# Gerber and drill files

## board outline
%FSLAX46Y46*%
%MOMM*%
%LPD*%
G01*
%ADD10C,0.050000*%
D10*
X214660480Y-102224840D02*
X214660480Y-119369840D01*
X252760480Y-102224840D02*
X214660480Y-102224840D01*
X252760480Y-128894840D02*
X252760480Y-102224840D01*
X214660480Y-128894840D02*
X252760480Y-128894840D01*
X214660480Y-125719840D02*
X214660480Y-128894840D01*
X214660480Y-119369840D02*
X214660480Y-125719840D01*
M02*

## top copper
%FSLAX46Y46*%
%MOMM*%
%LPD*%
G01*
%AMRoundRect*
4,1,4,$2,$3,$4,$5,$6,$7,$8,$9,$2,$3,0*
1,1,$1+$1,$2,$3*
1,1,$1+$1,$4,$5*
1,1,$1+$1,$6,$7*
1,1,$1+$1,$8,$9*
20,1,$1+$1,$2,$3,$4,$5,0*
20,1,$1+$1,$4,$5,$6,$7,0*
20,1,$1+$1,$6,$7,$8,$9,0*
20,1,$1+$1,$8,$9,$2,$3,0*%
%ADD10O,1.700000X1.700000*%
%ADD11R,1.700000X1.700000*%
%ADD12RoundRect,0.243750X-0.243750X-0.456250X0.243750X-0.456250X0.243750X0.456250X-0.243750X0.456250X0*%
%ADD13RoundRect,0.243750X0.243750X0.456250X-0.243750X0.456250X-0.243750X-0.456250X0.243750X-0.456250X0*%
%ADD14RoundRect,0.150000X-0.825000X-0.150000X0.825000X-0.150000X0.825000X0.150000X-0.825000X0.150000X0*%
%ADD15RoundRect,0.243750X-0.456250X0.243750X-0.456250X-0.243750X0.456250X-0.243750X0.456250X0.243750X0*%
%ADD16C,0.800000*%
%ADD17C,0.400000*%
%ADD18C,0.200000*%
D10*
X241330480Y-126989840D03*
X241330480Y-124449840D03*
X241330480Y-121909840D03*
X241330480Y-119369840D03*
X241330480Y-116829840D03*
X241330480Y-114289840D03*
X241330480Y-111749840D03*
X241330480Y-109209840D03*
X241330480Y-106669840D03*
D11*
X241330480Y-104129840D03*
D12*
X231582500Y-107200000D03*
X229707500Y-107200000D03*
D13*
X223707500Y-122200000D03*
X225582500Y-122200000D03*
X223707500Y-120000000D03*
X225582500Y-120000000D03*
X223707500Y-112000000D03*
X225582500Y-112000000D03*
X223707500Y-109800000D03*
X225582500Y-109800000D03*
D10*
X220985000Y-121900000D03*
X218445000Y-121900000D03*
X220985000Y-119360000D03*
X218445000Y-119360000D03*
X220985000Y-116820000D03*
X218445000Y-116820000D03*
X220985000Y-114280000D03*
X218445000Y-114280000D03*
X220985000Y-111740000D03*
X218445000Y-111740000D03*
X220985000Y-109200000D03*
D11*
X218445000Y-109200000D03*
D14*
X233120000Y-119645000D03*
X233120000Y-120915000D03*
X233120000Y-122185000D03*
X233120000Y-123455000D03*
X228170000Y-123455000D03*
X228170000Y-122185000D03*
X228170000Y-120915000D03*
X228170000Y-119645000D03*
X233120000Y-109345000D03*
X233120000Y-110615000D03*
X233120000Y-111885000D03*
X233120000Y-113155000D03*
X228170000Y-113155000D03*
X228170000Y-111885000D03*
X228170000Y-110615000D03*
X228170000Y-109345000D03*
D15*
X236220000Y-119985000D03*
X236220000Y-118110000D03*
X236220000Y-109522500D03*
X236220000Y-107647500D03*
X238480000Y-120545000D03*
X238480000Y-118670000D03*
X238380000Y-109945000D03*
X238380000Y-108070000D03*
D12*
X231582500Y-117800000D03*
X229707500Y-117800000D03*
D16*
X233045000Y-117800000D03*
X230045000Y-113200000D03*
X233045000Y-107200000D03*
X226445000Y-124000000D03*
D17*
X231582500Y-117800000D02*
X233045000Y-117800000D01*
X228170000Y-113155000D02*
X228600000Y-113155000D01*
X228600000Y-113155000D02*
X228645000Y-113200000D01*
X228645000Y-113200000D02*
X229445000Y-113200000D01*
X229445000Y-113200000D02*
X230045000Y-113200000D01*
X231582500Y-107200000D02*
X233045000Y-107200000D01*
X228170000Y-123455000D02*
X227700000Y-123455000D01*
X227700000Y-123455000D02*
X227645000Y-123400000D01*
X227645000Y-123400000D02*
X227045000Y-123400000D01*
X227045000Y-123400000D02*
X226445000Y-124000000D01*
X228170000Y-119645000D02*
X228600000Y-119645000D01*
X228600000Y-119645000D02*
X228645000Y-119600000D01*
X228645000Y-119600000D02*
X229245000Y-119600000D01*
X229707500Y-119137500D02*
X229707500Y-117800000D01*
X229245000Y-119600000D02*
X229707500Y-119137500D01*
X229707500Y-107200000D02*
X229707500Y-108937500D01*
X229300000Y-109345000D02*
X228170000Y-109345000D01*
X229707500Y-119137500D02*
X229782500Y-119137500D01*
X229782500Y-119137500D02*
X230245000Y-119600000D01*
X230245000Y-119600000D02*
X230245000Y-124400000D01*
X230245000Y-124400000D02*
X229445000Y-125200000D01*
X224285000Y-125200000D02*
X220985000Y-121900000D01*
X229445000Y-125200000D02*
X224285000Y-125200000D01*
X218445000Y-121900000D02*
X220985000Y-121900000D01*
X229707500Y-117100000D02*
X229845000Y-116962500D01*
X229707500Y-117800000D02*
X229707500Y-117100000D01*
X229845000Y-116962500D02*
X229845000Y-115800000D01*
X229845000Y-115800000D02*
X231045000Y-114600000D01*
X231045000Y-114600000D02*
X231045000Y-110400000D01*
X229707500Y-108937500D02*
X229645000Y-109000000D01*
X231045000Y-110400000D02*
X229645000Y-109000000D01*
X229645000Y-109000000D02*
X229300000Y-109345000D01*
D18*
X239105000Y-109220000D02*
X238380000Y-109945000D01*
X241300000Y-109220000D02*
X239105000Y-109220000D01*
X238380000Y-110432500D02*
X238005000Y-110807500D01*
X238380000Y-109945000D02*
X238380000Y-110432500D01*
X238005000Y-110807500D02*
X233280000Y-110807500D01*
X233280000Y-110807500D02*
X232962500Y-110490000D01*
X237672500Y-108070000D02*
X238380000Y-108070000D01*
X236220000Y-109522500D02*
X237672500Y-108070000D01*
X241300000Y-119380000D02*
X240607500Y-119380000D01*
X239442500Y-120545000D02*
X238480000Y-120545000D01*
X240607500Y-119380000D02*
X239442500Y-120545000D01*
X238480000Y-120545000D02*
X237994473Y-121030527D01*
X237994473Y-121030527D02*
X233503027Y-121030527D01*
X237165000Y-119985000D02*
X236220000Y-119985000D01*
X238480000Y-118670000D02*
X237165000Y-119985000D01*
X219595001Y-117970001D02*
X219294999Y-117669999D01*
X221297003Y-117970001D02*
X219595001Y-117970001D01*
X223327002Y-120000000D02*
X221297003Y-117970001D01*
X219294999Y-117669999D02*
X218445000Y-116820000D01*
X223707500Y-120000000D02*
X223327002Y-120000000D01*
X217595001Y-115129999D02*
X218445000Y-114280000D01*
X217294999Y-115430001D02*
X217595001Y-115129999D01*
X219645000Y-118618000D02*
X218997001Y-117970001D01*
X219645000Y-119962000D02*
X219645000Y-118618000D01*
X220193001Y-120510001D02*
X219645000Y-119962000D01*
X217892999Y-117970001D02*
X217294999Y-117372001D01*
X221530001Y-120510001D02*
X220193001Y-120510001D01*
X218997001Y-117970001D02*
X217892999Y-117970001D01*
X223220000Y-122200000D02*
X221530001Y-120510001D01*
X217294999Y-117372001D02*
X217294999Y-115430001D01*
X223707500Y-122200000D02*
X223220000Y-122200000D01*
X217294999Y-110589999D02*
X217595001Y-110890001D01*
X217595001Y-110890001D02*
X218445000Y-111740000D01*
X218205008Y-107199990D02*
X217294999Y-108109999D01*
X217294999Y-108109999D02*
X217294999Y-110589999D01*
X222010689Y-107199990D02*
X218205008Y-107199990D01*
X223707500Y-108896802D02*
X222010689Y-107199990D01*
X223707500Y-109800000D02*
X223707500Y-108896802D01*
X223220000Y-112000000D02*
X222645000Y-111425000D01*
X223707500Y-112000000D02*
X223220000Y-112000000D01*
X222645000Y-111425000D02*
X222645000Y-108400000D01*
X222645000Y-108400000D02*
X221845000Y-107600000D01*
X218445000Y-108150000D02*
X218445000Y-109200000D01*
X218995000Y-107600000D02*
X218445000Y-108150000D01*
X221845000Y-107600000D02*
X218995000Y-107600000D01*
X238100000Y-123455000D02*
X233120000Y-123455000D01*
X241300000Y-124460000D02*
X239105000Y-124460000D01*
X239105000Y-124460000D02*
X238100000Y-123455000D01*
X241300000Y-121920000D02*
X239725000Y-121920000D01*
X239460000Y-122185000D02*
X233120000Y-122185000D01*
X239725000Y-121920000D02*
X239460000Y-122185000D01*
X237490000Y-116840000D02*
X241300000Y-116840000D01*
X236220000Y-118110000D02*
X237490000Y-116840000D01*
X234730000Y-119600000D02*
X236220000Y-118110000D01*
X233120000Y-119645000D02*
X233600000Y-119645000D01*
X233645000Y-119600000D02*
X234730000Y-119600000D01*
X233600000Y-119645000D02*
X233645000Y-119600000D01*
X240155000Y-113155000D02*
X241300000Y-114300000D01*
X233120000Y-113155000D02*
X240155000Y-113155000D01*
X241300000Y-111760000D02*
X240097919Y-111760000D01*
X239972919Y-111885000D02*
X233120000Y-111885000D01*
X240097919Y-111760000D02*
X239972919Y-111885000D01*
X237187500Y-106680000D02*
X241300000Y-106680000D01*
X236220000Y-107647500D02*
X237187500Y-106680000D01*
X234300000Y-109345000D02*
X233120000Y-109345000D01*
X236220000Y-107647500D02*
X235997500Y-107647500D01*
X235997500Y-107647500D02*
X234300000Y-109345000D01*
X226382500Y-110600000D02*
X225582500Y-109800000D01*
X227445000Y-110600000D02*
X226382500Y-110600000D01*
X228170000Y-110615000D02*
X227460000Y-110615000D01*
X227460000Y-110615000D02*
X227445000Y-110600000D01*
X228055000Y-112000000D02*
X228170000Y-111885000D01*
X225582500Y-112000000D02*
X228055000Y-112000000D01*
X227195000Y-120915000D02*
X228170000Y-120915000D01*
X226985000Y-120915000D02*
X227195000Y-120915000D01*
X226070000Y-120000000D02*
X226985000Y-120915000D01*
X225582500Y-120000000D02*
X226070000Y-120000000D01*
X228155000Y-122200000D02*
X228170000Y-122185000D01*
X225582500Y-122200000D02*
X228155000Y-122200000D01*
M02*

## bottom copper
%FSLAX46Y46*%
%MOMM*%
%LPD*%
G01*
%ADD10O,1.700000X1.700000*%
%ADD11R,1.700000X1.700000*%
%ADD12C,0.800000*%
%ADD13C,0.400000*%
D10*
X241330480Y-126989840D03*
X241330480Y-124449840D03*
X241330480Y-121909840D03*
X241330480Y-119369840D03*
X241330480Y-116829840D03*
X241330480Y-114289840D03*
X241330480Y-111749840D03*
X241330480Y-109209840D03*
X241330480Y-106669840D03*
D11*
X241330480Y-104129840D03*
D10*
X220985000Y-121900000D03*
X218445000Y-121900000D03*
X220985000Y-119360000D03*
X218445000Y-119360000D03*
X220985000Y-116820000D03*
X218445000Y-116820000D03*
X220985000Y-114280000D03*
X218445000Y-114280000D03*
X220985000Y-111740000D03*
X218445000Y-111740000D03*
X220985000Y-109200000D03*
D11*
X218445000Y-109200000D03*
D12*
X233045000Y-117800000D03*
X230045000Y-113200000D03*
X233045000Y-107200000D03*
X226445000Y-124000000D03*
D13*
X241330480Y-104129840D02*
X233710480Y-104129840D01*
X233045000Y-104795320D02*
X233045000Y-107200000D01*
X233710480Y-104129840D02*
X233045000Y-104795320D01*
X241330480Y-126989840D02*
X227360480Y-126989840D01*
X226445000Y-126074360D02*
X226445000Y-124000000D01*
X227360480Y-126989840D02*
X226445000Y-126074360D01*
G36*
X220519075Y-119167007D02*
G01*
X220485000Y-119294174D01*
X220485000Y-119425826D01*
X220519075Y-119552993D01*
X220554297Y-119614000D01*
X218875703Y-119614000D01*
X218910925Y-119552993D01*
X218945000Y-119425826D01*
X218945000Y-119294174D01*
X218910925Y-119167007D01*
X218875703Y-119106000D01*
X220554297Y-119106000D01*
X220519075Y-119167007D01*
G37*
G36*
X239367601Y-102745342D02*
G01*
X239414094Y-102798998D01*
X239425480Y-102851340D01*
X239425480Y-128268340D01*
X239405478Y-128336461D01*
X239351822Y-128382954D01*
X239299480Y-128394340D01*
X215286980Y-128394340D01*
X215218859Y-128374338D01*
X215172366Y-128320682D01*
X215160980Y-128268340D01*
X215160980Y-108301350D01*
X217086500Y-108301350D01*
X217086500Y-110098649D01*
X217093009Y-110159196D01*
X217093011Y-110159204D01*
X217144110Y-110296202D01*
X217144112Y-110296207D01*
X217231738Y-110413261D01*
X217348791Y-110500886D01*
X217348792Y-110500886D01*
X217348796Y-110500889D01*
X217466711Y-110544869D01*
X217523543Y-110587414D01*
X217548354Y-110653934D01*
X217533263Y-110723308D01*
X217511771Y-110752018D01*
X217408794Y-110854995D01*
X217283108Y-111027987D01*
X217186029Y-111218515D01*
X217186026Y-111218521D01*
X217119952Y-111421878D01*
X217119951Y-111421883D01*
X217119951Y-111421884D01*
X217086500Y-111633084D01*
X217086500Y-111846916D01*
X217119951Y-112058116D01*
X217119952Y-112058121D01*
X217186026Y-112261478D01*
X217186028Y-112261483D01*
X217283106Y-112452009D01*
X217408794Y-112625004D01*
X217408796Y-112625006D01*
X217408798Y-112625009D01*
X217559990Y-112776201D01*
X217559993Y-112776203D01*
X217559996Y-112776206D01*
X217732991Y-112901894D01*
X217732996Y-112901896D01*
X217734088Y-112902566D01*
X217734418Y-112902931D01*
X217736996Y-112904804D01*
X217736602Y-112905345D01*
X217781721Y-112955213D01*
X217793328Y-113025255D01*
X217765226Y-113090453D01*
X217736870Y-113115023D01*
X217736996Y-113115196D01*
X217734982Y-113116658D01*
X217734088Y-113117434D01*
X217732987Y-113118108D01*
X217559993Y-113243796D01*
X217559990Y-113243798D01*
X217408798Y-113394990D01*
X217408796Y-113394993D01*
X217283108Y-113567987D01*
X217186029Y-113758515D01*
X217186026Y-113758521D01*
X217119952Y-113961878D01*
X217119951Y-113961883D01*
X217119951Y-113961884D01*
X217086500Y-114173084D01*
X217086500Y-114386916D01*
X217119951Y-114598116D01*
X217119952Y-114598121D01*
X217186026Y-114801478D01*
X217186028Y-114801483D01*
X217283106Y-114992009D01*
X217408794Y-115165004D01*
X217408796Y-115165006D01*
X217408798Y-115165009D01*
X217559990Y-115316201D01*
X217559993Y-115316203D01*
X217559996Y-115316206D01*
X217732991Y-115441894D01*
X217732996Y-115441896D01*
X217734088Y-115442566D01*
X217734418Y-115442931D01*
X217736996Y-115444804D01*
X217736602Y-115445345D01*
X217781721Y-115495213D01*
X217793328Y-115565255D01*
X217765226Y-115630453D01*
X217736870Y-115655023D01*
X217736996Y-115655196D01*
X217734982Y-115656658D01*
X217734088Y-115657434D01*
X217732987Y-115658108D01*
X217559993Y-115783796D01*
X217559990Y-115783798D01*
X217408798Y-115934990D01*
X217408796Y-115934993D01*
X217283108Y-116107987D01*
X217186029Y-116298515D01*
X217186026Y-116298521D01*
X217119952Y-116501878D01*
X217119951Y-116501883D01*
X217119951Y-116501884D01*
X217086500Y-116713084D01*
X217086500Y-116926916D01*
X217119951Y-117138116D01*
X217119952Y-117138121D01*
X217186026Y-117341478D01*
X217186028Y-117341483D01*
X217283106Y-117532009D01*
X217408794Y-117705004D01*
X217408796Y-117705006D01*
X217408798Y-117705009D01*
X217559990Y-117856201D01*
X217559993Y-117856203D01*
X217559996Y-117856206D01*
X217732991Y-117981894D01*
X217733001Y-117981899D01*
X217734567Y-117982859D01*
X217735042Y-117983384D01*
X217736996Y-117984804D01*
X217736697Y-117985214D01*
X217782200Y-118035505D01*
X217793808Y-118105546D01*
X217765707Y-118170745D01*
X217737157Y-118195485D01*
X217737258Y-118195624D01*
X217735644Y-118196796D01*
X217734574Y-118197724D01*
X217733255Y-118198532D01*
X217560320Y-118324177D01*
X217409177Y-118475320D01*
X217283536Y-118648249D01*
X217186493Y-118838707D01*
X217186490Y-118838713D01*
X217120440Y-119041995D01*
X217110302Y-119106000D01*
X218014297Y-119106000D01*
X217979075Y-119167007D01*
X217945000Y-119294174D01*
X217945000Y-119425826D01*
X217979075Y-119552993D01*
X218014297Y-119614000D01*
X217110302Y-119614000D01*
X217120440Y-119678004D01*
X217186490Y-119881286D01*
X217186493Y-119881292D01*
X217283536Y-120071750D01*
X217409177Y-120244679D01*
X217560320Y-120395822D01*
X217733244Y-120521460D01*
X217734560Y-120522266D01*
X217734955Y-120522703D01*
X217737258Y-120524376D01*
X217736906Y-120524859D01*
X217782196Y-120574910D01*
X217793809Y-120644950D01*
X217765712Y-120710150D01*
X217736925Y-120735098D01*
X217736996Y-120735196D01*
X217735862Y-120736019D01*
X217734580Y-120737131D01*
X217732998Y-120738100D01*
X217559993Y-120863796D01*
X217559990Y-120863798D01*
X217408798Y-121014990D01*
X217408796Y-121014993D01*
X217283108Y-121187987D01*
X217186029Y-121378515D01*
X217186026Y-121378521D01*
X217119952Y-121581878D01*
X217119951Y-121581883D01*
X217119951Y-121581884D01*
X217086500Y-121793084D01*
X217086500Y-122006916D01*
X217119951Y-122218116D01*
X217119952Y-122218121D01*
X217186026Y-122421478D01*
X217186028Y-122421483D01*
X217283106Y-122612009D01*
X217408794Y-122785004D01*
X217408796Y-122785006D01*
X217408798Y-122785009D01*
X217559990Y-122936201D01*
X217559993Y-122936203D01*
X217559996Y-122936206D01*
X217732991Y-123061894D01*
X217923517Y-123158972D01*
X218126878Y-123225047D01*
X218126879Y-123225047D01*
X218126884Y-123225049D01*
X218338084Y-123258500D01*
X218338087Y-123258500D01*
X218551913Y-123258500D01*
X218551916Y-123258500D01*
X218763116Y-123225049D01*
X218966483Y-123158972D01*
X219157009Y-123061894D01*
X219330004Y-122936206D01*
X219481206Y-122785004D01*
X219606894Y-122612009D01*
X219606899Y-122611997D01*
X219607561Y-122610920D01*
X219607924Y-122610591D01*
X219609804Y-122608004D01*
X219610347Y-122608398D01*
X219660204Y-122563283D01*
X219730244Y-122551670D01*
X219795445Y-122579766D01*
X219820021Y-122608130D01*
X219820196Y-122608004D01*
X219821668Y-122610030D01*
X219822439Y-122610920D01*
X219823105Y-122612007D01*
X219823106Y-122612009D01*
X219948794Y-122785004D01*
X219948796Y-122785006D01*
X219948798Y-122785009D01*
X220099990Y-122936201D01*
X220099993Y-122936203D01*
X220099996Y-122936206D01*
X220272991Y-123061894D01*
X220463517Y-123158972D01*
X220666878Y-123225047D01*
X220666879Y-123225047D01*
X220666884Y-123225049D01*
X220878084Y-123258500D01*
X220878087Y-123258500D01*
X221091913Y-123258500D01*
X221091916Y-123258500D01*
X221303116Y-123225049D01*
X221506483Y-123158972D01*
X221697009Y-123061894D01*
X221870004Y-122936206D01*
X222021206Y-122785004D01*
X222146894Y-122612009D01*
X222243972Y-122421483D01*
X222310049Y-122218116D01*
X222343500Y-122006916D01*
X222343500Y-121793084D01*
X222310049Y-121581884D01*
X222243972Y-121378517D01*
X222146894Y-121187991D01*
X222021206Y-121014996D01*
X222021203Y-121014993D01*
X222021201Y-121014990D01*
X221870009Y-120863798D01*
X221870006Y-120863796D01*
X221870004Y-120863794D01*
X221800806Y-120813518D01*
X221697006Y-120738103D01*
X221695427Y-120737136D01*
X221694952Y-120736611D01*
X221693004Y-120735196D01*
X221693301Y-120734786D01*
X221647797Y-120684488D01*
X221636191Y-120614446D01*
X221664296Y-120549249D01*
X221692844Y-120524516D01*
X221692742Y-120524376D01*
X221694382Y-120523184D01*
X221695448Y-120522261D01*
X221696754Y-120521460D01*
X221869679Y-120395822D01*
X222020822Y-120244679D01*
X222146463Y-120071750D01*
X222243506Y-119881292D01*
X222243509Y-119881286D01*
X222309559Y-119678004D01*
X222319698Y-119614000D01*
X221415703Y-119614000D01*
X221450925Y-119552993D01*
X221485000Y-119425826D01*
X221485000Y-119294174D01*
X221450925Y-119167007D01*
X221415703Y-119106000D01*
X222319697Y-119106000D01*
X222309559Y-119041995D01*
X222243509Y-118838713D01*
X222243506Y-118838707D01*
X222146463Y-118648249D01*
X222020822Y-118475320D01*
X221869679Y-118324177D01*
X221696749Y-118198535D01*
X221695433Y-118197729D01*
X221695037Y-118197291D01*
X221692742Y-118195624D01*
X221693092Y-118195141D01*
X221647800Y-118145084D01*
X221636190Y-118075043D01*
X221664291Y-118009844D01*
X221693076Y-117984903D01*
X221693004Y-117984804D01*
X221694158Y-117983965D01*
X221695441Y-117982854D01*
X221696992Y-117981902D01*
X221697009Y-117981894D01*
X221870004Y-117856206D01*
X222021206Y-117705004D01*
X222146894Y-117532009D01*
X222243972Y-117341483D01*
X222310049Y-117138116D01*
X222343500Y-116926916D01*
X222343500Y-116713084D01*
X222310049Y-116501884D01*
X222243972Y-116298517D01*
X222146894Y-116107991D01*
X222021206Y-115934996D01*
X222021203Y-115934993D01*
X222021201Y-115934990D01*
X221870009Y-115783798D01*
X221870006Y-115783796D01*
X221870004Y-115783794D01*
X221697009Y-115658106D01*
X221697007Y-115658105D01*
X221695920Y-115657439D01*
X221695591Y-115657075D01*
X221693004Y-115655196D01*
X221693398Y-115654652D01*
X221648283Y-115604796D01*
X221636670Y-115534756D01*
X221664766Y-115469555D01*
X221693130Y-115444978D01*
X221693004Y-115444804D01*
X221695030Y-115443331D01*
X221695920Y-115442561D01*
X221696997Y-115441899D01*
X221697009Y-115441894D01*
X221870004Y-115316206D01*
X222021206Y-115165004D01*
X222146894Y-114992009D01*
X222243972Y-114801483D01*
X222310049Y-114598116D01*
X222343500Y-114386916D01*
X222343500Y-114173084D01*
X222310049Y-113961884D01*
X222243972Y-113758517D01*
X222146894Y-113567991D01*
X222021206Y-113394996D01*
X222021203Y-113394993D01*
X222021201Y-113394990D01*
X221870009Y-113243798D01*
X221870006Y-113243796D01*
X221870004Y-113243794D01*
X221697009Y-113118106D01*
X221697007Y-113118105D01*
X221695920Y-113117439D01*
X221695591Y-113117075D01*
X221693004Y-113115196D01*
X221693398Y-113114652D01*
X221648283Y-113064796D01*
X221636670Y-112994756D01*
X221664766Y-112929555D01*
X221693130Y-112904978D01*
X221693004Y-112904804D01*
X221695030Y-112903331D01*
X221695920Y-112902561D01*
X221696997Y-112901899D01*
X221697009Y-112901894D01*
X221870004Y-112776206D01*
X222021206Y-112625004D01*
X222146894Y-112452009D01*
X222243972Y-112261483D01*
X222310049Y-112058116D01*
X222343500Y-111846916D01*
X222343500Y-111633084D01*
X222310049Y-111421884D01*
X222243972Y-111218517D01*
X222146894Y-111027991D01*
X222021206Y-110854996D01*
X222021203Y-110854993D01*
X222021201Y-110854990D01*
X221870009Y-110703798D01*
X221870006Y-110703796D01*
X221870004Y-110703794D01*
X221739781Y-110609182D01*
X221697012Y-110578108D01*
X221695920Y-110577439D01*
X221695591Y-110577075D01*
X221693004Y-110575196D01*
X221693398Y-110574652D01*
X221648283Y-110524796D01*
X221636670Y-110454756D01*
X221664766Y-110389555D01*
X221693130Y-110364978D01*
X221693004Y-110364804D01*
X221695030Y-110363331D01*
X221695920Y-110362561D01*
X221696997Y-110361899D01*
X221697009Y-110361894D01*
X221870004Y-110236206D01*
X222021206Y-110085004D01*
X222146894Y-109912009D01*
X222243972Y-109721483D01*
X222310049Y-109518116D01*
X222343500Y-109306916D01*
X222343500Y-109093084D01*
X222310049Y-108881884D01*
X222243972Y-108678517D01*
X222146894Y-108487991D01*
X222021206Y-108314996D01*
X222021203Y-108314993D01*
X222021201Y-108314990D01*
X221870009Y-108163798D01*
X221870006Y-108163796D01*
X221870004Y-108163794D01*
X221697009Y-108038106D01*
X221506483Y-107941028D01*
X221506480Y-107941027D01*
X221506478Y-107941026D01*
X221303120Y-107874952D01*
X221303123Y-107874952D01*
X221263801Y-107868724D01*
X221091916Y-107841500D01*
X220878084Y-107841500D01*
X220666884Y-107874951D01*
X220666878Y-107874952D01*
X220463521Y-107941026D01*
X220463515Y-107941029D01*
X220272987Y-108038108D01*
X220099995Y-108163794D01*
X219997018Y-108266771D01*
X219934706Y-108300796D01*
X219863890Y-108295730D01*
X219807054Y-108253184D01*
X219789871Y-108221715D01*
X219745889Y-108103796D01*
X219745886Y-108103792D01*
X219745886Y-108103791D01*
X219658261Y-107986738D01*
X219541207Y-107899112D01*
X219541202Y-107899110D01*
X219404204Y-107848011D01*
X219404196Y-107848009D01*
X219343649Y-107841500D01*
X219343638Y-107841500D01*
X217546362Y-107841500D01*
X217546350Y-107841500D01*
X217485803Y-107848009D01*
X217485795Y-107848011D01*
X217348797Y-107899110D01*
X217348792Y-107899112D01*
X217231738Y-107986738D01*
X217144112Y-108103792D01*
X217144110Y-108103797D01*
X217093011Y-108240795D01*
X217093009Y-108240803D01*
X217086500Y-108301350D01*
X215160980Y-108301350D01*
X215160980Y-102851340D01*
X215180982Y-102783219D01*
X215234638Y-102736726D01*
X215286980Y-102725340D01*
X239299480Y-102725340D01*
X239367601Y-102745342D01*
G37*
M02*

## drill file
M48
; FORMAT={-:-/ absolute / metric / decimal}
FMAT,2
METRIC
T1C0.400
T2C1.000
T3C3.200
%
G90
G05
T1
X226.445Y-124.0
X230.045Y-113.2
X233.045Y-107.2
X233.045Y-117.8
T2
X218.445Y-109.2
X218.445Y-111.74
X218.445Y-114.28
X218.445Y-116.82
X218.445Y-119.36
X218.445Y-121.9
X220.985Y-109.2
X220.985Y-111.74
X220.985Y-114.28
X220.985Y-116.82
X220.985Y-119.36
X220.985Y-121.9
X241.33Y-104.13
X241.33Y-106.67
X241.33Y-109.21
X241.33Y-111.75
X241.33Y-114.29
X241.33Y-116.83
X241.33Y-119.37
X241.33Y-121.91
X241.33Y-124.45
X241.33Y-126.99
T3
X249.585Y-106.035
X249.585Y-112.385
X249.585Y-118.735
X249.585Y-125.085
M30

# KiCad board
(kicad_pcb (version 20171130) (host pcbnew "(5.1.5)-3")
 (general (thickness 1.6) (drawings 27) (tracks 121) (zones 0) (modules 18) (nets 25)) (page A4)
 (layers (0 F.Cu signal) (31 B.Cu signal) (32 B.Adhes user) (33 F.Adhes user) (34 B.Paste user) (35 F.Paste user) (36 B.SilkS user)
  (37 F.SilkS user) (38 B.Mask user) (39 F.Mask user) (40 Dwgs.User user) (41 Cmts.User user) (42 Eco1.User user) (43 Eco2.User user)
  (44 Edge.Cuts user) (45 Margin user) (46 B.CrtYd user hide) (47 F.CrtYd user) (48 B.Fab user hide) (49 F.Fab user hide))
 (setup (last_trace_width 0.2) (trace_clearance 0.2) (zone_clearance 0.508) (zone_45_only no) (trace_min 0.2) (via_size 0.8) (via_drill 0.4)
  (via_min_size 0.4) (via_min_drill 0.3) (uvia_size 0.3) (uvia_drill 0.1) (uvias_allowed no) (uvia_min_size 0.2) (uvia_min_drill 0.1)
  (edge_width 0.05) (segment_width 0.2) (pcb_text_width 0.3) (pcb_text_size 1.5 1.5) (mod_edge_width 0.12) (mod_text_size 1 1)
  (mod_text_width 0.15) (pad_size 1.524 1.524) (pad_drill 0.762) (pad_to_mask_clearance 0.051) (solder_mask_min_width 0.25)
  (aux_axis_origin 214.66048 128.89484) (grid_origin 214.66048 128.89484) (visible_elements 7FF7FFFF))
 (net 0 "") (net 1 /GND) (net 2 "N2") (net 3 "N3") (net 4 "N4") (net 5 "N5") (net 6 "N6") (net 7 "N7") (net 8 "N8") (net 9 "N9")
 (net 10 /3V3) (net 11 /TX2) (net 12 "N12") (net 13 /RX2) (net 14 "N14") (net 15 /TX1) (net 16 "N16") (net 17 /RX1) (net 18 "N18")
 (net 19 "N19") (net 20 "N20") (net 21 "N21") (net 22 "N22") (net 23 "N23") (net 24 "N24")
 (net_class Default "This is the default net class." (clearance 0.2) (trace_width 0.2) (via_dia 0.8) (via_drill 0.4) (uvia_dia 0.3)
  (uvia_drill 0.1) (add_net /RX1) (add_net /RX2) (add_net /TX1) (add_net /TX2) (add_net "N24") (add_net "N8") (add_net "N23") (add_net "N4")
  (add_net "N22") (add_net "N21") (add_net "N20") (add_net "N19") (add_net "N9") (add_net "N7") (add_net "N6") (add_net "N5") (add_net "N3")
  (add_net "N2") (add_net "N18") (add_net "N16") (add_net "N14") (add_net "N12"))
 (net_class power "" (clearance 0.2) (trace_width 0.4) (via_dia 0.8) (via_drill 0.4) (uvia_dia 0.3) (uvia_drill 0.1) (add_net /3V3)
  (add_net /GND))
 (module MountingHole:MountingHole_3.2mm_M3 (layer F.Cu) (at 249.58548 118.73484)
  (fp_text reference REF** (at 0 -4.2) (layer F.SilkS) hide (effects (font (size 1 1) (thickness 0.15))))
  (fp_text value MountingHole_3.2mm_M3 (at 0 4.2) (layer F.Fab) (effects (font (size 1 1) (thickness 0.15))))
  (pad 1 np_thru_hole circle (at 0 0) (size 3.2 3.2) (drill 3.2) (layers *.Cu *.Mask)))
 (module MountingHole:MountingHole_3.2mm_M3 (layer F.Cu) (at 249.58548 125.08484)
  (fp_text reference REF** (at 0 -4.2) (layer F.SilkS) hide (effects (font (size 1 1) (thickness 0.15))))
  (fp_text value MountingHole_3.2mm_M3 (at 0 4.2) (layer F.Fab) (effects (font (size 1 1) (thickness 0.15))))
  (pad 1 np_thru_hole circle (at 0 0) (size 3.2 3.2) (drill 3.2) (layers *.Cu *.Mask)))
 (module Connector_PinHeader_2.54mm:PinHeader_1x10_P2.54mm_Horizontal (layer F.Cu) (at 241.33048 104.12984)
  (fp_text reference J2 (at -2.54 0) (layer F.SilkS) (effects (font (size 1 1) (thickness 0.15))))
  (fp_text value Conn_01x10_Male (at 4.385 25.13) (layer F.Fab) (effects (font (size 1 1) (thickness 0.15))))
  (pad 10 thru_hole oval (at 0 22.86) (size 1.7 1.7) (drill 1) (layers *.Cu *.Mask) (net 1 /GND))
  (pad 9 thru_hole oval (at 0 20.32) (size 1.7 1.7) (drill 1) (layers *.Cu *.Mask) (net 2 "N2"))
  (pad 8 thru_hole oval (at 0 17.78) (size 1.7 1.7) (drill 1) (layers *.Cu *.Mask) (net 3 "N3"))
  (pad 7 thru_hole oval (at 0 15.24) (size 1.7 1.7) (drill 1) (layers *.Cu *.Mask) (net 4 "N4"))
  (pad 6 thru_hole oval (at 0 12.7) (size 1.7 1.7) (drill 1) (layers *.Cu *.Mask) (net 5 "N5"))
  (pad 5 thru_hole oval (at 0 10.16) (size 1.7 1.7) (drill 1) (layers *.Cu *.Mask) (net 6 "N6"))
  (pad 4 thru_hole oval (at 0 7.62) (size 1.7 1.7) (drill 1) (layers *.Cu *.Mask) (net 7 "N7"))
  (pad 3 thru_hole oval (at 0 5.08) (size 1.7 1.7) (drill 1) (layers *.Cu *.Mask) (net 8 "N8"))
  (pad 2 thru_hole oval (at 0 2.54) (size 1.7 1.7) (drill 1) (layers *.Cu *.Mask) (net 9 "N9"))
  (pad 1 thru_hole rect (at 0 0) (size 1.7 1.7) (drill 1) (layers *.Cu *.Mask) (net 1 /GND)))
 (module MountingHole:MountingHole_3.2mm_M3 (layer F.Cu) (at 249.58548 112.38484)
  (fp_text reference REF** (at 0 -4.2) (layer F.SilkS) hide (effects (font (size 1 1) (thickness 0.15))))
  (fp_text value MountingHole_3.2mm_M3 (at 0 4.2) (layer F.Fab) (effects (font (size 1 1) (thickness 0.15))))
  (pad 1 np_thru_hole circle (at 0 0) (size 3.2 3.2) (drill 3.2) (layers *.Cu *.Mask)))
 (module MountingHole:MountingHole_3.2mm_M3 (layer F.Cu) (at 249.58548 106.03484)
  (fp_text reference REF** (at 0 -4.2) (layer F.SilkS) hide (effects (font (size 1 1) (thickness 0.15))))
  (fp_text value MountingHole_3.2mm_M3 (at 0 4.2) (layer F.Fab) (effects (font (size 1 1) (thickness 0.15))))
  (pad 1 np_thru_hole circle (at 0 0) (size 3.2 3.2) (drill 3.2) (layers *.Cu *.Mask)))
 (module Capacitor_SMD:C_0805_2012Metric (layer F.Cu) (at 230.645 107.2)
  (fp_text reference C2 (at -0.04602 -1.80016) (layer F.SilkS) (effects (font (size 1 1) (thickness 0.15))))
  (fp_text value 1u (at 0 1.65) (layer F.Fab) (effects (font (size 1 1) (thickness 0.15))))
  (pad 2 smd roundrect (at 0.9375 0) (size 0.975 1.4) (layers F.Cu F.Paste F.Mask) (roundrect_rratio 0.25) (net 1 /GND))
  (pad 1 smd roundrect (at -0.9375 0) (size 0.975 1.4) (layers F.Cu F.Paste F.Mask) (roundrect_rratio 0.25) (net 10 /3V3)))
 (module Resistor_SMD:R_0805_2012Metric (layer F.Cu) (at 224.645 122.2 180)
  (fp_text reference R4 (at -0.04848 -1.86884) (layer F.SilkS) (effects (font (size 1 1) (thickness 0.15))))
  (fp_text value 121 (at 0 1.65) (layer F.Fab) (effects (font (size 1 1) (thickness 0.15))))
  (pad 2 smd roundrect (at 0.9375 0 180) (size 0.975 1.4) (layers F.Cu F.Paste F.Mask) (roundrect_rratio 0.25) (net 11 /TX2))
  (pad 1 smd roundrect (at -0.9375 0 180) (size 0.975 1.4) (layers F.Cu F.Paste F.Mask) (roundrect_rratio 0.25) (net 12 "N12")))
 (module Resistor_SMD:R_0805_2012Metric (layer F.Cu) (at 224.645 120 180)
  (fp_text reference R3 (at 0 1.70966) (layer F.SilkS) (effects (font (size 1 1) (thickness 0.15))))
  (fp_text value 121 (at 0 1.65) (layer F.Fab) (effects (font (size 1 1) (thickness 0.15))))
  (pad 2 smd roundrect (at 0.9375 0 180) (size 0.975 1.4) (layers F.Cu F.Paste F.Mask) (roundrect_rratio 0.25) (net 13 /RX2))
  (pad 1 smd roundrect (at -0.9375 0 180) (size 0.975 1.4) (layers F.Cu F.Paste F.Mask) (roundrect_rratio 0.25) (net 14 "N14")))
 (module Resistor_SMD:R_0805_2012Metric (layer F.Cu) (at 224.645 112 180)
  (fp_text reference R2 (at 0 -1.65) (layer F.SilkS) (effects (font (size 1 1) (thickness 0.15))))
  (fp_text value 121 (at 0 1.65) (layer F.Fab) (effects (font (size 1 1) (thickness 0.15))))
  (pad 2 smd roundrect (at 0.9375 0 180) (size 0.975 1.4) (layers F.Cu F.Paste F.Mask) (roundrect_rratio 0.25) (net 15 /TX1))
  (pad 1 smd roundrect (at -0.9375 0 180) (size 0.975 1.4) (layers F.Cu F.Paste F.Mask) (roundrect_rratio 0.25) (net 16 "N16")))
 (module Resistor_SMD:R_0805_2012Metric (layer F.Cu) (at 224.645 109.8 180)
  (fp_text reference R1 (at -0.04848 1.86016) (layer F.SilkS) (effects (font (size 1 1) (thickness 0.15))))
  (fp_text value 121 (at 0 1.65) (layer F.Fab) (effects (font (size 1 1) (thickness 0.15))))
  (pad 2 smd roundrect (at 0.9375 0 180) (size 0.975 1.4) (layers F.Cu F.Paste F.Mask) (roundrect_rratio 0.25) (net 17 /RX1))
  (pad 1 smd roundrect (at -0.9375 0 180) (size 0.975 1.4) (layers F.Cu F.Paste F.Mask) (roundrect_rratio 0.25) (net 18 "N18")))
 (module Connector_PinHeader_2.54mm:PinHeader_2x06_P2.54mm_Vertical (layer F.Cu) (at 218.445 109.2)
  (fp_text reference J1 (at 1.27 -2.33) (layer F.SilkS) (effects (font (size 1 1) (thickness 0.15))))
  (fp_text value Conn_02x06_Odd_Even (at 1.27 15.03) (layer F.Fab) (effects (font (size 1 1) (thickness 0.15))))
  (pad 12 thru_hole oval (at 2.54 12.7) (size 1.7 1.7) (drill 1) (layers *.Cu *.Mask) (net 10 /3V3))
  (pad 11 thru_hole oval (at 0 12.7) (size 1.7 1.7) (drill 1) (layers *.Cu *.Mask) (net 10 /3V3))
  (pad 10 thru_hole oval (at 2.54 10.16) (size 1.7 1.7) (drill 1) (layers *.Cu *.Mask) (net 1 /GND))
  (pad 9 thru_hole oval (at 0 10.16) (size 1.7 1.7) (drill 1) (layers *.Cu *.Mask) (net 1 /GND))
  (pad 8 thru_hole oval (at 2.54 7.62) (size 1.7 1.7) (drill 1) (layers *.Cu *.Mask) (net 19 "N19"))
  (pad 7 thru_hole oval (at 0 7.62) (size 1.7 1.7) (drill 1) (layers *.Cu *.Mask) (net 13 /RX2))
  (pad 6 thru_hole oval (at 2.54 5.08) (size 1.7 1.7) (drill 1) (layers *.Cu *.Mask) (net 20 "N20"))
  (pad 5 thru_hole oval (at 0 5.08) (size 1.7 1.7) (drill 1) (layers *.Cu *.Mask) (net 11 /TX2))
  (pad 4 thru_hole oval (at 2.54 2.54) (size 1.7 1.7) (drill 1) (layers *.Cu *.Mask) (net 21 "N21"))
  (pad 3 thru_hole oval (at 0 2.54) (size 1.7 1.7) (drill 1) (layers *.Cu *.Mask) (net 17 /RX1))
  (pad 2 thru_hole oval (at 2.54 0) (size 1.7 1.7) (drill 1) (layers *.Cu *.Mask) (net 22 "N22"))
  (pad 1 thru_hole rect (at 0 0) (size 1.7 1.7) (drill 1) (layers *.Cu *.Mask) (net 15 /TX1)))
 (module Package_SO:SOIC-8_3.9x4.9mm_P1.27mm (layer F.Cu) (at 230.645 121.55)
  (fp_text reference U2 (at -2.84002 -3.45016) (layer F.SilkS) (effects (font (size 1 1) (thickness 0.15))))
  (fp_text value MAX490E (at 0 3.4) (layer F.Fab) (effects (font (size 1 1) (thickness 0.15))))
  (pad 8 smd roundrect (at 2.475 -1.905) (size 1.95 0.6) (layers F.Cu F.Paste F.Mask) (roundrect_rratio 0.25) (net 5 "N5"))
  (pad 7 smd roundrect (at 2.475 -0.635) (size 1.95 0.6) (layers F.Cu F.Paste F.Mask) (roundrect_rratio 0.25) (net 4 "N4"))
  (pad 6 smd roundrect (at 2.475 0.635) (size 1.95 0.6) (layers F.Cu F.Paste F.Mask) (roundrect_rratio 0.25) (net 3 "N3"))
  (pad 5 smd roundrect (at 2.475 1.905) (size 1.95 0.6) (layers F.Cu F.Paste F.Mask) (roundrect_rratio 0.25) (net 2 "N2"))
  (pad 4 smd roundrect (at -2.475 1.905) (size 1.95 0.6) (layers F.Cu F.Paste F.Mask) (roundrect_rratio 0.25) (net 1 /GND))
  (pad 3 smd roundrect (at -2.475 0.635) (size 1.95 0.6) (layers F.Cu F.Paste F.Mask) (roundrect_rratio 0.25) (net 12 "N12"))
  (pad 2 smd roundrect (at -2.475 -0.635) (size 1.95 0.6) (layers F.Cu F.Paste F.Mask) (roundrect_rratio 0.25) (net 14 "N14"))
  (pad 1 smd roundrect (at -2.475 -1.905) (size 1.95 0.6) (layers F.Cu F.Paste F.Mask) (roundrect_rratio 0.25) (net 10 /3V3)))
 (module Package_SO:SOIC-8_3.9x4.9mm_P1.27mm (layer F.Cu) (at 230.645 111.25)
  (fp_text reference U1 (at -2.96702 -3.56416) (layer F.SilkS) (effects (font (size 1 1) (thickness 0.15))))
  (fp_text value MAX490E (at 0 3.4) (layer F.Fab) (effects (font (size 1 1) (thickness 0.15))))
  (pad 8 smd roundrect (at 2.475 -1.905) (size 1.95 0.6) (layers F.Cu F.Paste F.Mask) (roundrect_rratio 0.25) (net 9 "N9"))
  (pad 7 smd roundrect (at 2.475 -0.635) (size 1.95 0.6) (layers F.Cu F.Paste F.Mask) (roundrect_rratio 0.25) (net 8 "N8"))
  (pad 6 smd roundrect (at 2.475 0.635) (size 1.95 0.6) (layers F.Cu F.Paste F.Mask) (roundrect_rratio 0.25) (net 7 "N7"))
  (pad 5 smd roundrect (at 2.475 1.905) (size 1.95 0.6) (layers F.Cu F.Paste F.Mask) (roundrect_rratio 0.25) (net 6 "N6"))
  (pad 4 smd roundrect (at -2.475 1.905) (size 1.95 0.6) (layers F.Cu F.Paste F.Mask) (roundrect_rratio 0.25) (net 1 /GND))
  (pad 3 smd roundrect (at -2.475 0.635) (size 1.95 0.6) (layers F.Cu F.Paste F.Mask) (roundrect_rratio 0.25) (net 16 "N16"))
  (pad 2 smd roundrect (at -2.475 -0.635) (size 1.95 0.6) (layers F.Cu F.Paste F.Mask) (roundrect_rratio 0.25) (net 18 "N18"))
  (pad 1 smd roundrect (at -2.475 -1.905) (size 1.95 0.6) (layers F.Cu F.Paste F.Mask) (roundrect_rratio 0.25) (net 10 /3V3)))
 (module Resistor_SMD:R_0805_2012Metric (layer F.Cu) (at 236.22 119.0475 270)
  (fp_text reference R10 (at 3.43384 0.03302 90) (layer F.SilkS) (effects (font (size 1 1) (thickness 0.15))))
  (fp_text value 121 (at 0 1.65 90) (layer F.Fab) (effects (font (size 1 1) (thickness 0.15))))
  (pad 2 smd roundrect (at 0.9375 0 270) (size 0.975 1.4) (layers F.Cu F.Paste F.Mask) (roundrect_rratio 0.25) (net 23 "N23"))
  (pad 1 smd roundrect (at -0.9375 0 270) (size 0.975 1.4) (layers F.Cu F.Paste F.Mask) (roundrect_rratio 0.25) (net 5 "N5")))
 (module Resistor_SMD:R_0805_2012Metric (layer F.Cu) (at 236.22 108.585 270)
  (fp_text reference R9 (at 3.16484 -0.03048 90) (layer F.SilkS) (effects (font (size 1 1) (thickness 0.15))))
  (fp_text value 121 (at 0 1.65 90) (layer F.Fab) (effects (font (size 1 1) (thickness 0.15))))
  (pad 2 smd roundrect (at 0.9375 0 270) (size 0.975 1.4) (layers F.Cu F.Paste F.Mask) (roundrect_rratio 0.25) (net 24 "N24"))
  (pad 1 smd roundrect (at -0.9375 0 270) (size 0.975 1.4) (layers F.Cu F.Paste F.Mask) (roundrect_rratio 0.25) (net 9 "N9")))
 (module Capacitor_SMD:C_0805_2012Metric (layer F.Cu) (at 238.48 119.6075 270)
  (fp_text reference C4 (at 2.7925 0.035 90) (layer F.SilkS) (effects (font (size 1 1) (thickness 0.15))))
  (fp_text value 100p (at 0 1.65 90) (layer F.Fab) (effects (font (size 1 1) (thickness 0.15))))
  (pad 2 smd roundrect (at 0.9375 0 270) (size 0.975 1.4) (layers F.Cu F.Paste F.Mask) (roundrect_rratio 0.25) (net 4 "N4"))
  (pad 1 smd roundrect (at -0.9375 0 270) (size 0.975 1.4) (layers F.Cu F.Paste F.Mask) (roundrect_rratio 0.25) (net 23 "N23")))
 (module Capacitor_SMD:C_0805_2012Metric (layer F.Cu) (at 238.38 109.0075 270)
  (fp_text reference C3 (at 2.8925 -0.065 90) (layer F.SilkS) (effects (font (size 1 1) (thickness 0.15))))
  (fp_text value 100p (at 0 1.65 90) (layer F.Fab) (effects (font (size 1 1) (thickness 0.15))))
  (pad 2 smd roundrect (at 0.9375 0 270) (size 0.975 1.4) (layers F.Cu F.Paste F.Mask) (roundrect_rratio 0.25) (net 8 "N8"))
  (pad 1 smd roundrect (at -0.9375 0 270) (size 0.975 1.4) (layers F.Cu F.Paste F.Mask) (roundrect_rratio 0.25) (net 24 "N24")))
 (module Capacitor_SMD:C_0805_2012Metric (layer F.Cu) (at 230.645 117.8)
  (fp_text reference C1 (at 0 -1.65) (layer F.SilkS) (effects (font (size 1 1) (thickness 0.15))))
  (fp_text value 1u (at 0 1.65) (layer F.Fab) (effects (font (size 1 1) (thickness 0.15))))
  (pad 2 smd roundrect (at 0.9375 0) (size 0.975 1.4) (layers F.Cu F.Paste F.Mask) (roundrect_rratio 0.25) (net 1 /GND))
  (pad 1 smd roundrect (at -0.9375 0) (size 0.975 1.4) (layers F.Cu F.Paste F.Mask) (roundrect_rratio 0.25) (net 10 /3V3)))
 (gr_line (start 214.66048 102.22484) (end 214.66048 119.36984) (layer Edge.Cuts) (width 0.05))
 (gr_line (start 252.76048 102.22484) (end 214.66048 102.22484) (layer Edge.Cuts) (width 0.05))
 (gr_line (start 252.76048 128.89484) (end 252.76048 102.22484) (layer Edge.Cuts) (width 0.05))
 (gr_line (start 214.66048 128.89484) (end 252.76048 128.89484) (layer Edge.Cuts) (width 0.05))
 (gr_line (start 214.66048 125.71984) (end 214.66048 128.89484) (layer Edge.Cuts) (width 0.05))
 (gr_line (start 214.66048 119.36984) (end 214.66048 125.71984) (layer Edge.Cuts) (width 0.05))
 (via (at 233.045 117.8) (size 0.8) (drill 0.4) (layers F.Cu B.Cu) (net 1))
 (segment (start 231.5825 117.8) (end 233.045 117.8) (width 0.4) (layer F.Cu) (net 1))
 (segment (start 228.17 113.155) (end 228.6 113.155) (width 0.4) (layer F.Cu) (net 1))
 (segment (start 228.6 113.155) (end 228.645 113.2) (width 0.4) (layer F.Cu) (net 1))
 (segment (start 228.645 113.2) (end 229.445 113.2) (width 0.4) (layer F.Cu) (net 1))
 (via (at 230.045 113.2) (size 0.8) (drill 0.4) (layers F.Cu B.Cu) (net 1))
 (segment (start 229.445 113.2) (end 230.045 113.2) (width 0.4) (layer F.Cu) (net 1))
 (via (at 233.045 107.2) (size 0.8) (drill 0.4) (layers F.Cu B.Cu) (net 1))
 (segment (start 231.5825 107.2) (end 233.045 107.2) (width 0.4) (layer F.Cu) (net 1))
 (segment (start 228.17 123.455) (end 227.7 123.455) (width 0.4) (layer F.Cu) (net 1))
 (segment (start 227.7 123.455) (end 227.645 123.4) (width 0.4) (layer F.Cu) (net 1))
 (via (at 226.445 124) (size 0.8) (drill 0.4) (layers F.Cu B.Cu) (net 1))
 (segment (start 227.645 123.4) (end 227.045 123.4) (width 0.4) (layer F.Cu) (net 1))
 (segment (start 227.045 123.4) (end 226.445 124) (width 0.4) (layer F.Cu) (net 1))
 (segment (start 241.33048 104.12984) (end 233.71048 104.12984) (width 0.4) (layer B.Cu) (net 1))
 (segment (start 233.045 104.79532) (end 233.045 107.2) (width 0.4) (layer B.Cu) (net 1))
 (segment (start 233.71048 104.12984) (end 233.045 104.79532) (width 0.4) (layer B.Cu) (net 1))
 (segment (start 241.33048 126.98984) (end 227.36048 126.98984) (width 0.4) (layer B.Cu) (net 1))
 (segment (start 226.445 126.07436) (end 226.445 124) (width 0.4) (layer B.Cu) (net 1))
 (segment (start 227.36048 126.98984) (end 226.445 126.07436) (width 0.4) (layer B.Cu) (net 1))
 (segment (start 228.17 119.645) (end 228.6 119.645) (width 0.4) (layer F.Cu) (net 10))
 (segment (start 228.6 119.645) (end 228.645 119.6) (width 0.4) (layer F.Cu) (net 10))
 (segment (start 228.645 119.6) (end 229.245 119.6) (width 0.4) (layer F.Cu) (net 10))
 (segment (start 229.7075 119.1375) (end 229.7075 117.8) (width 0.4) (layer F.Cu) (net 10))
 (segment (start 229.245 119.6) (end 229.7075 119.1375) (width 0.4) (layer F.Cu) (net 10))
 (segment (start 229.7075 107.2) (end 229.7075 108.9375) (width 0.4) (layer F.Cu) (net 10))
 (segment (start 229.3 109.345) (end 228.17 109.345) (width 0.4) (layer F.Cu) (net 10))
 (segment (start 229.7075 119.1375) (end 229.7825 119.1375) (width 0.4) (layer F.Cu) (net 10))
 (segment (start 229.7825 119.1375) (end 230.245 119.6) (width 0.4) (layer F.Cu) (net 10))
 (segment (start 230.245 119.6) (end 230.245 124.4) (width 0.4) (layer F.Cu) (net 10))
 (segment (start 230.245 124.4) (end 229.445 125.2) (width 0.4) (layer F.Cu) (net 10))
 (segment (start 224.285 125.2) (end 220.985 121.9) (width 0.4) (layer F.Cu) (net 10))
 (segment (start 229.445 125.2) (end 224.285 125.2) (width 0.4) (layer F.Cu) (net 10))
 (segment (start 218.445 121.9) (end 220.985 121.9) (width 0.4) (layer F.Cu) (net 10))
 (segment (start 229.7075 117.1) (end 229.845 116.9625) (width 0.4) (layer F.Cu) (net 10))
 (segment (start 229.7075 117.8) (end 229.7075 117.1) (width 0.4) (layer F.Cu) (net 10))
 (segment (start 229.845 116.9625) (end 229.845 115.8) (width 0.4) (layer F.Cu) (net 10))
 (segment (start 229.845 115.8) (end 231.045 114.6) (width 0.4) (layer F.Cu) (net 10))
 (segment (start 231.045 114.6) (end 231.045 110.4) (width 0.4) (layer F.Cu) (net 10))
 (segment (start 229.7075 108.9375) (end 229.645 109) (width 0.4) (layer F.Cu) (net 10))
 (segment (start 231.045 110.4) (end 229.645 109) (width 0.4) (layer F.Cu) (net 10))
 (segment (start 229.645 109) (end 229.3 109.345) (width 0.4) (layer F.Cu) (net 10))
 (segment (start 239.105 109.22) (end 238.38 109.945) (width 0.2) (layer F.Cu) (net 8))
 (segment (start 241.3 109.22) (end 239.105 109.22) (width 0.2) (layer F.Cu) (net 8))
 (segment (start 238.38 110.4325) (end 238.005 110.8075) (width 0.2) (layer F.Cu) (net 8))
 (segment (start 238.38 109.945) (end 238.38 110.4325) (width 0.2) (layer F.Cu) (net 8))
 (segment (start 238.005 110.8075) (end 233.28 110.8075) (width 0.2) (layer F.Cu) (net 8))
 (segment (start 233.28 110.8075) (end 232.9625 110.49) (width 0.2) (layer F.Cu) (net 8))
 (segment (start 237.6725 108.07) (end 238.38 108.07) (width 0.2) (layer F.Cu) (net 24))
 (segment (start 236.22 109.5225) (end 237.6725 108.07) (width 0.2) (layer F.Cu) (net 24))
 (segment (start 241.3 119.38) (end 240.6075 119.38) (width 0.2) (layer F.Cu) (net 4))
 (segment (start 239.4425 120.545) (end 238.48 120.545) (width 0.2) (layer F.Cu) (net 4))
 (segment (start 240.6075 119.38) (end 239.4425 120.545) (width 0.2) (layer F.Cu) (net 4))
 (segment (start 238.48 120.545) (end 237.994473 121.030527) (width 0.2) (layer F.Cu) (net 4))
 (segment (start 237.994473 121.030527) (end 233.503027 121.030527) (width 0.2) (layer F.Cu) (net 4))
 (segment (start 237.165 119.985) (end 236.22 119.985) (width 0.2) (layer F.Cu) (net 23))
 (segment (start 238.48 118.67) (end 237.165 119.985) (width 0.2) (layer F.Cu) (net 23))
 (segment (start 219.595001 117.970001) (end 219.294999 117.669999) (width 0.2) (layer F.Cu) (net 13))
 (segment (start 221.297003 117.970001) (end 219.595001 117.970001) (width 0.2) (layer F.Cu) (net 13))
 (segment (start 223.327002 120) (end 221.297003 117.970001) (width 0.2) (layer F.Cu) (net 13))
 (segment (start 219.294999 117.669999) (end 218.445 116.82) (width 0.2) (layer F.Cu) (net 13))
 (segment (start 223.7075 120) (end 223.327002 120) (width 0.2) (layer F.Cu) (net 13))
 (segment (start 217.595001 115.129999) (end 218.445 114.28) (width 0.2) (layer F.Cu) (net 11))
 (segment (start 217.294999 115.430001) (end 217.595001 115.129999) (width 0.2) (layer F.Cu) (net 11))
 (segment (start 219.645 118.618) (end 218.997001 117.970001) (width 0.2) (layer F.Cu) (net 11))
 (segment (start 219.645 119.962) (end 219.645 118.618) (width 0.2) (layer F.Cu) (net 11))
 (segment (start 220.193001 120.510001) (end 219.645 119.962) (width 0.2) (layer F.Cu) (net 11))
 (segment (start 217.892999 117.970001) (end 217.294999 117.372001) (width 0.2) (layer F.Cu) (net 11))
 (segment (start 221.530001 120.510001) (end 220.193001 120.510001) (width 0.2) (layer F.Cu) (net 11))
 (segment (start 218.997001 117.970001) (end 217.892999 117.970001) (width 0.2) (layer F.Cu) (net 11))
 (segment (start 223.22 122.2) (end 221.530001 120.510001) (width 0.2) (layer F.Cu) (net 11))
 (segment (start 217.294999 117.372001) (end 217.294999 115.430001) (width 0.2) (layer F.Cu) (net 11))
 (segment (start 223.7075 122.2) (end 223.22 122.2) (width 0.2) (layer F.Cu) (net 11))
 (segment (start 217.294999 110.589999) (end 217.595001 110.890001) (width 0.2) (layer F.Cu) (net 17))
 (segment (start 217.595001 110.890001) (end 218.445 111.74) (width 0.2) (layer F.Cu) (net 17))
 (segment (start 218.205008 107.19999) (end 217.294999 108.109999) (width 0.2) (layer F.Cu) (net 17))
 (segment (start 217.294999 108.109999) (end 217.294999 110.589999) (width 0.2) (layer F.Cu) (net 17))
 (segment (start 222.010689 107.19999) (end 218.205008 107.19999) (width 0.2) (layer F.Cu) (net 17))
 (segment (start 223.7075 108.896802) (end 222.010689 107.19999) (width 0.2) (layer F.Cu) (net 17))
 (segment (start 223.7075 109.8) (end 223.7075 108.896802) (width 0.2) (layer F.Cu) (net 17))
 (segment (start 223.22 112) (end 222.645 111.425) (width 0.2) (layer F.Cu) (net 15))
 (segment (start 223.7075 112) (end 223.22 112) (width 0.2) (layer F.Cu) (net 15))
 (segment (start 222.645 111.425) (end 222.645 108.4) (width 0.2) (layer F.Cu) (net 15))
 (segment (start 222.645 108.4) (end 221.845 107.6) (width 0.2) (layer F.Cu) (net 15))
 (segment (start 218.445 108.15) (end 218.445 109.2) (width 0.2) (layer F.Cu) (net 15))
 (segment (start 218.995 107.6) (end 218.445 108.15) (width 0.2) (layer F.Cu) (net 15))
 (segment (start 221.845 107.6) (end 218.995 107.6) (width 0.2) (layer F.Cu) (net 15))
 (segment (start 238.1 123.455) (end 233.12 123.455) (width 0.2) (layer F.Cu) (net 2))
 (segment (start 241.3 124.46) (end 239.105 124.46) (width 0.2) (layer F.Cu) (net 2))
 (segment (start 239.105 124.46) (end 238.1 123.455) (width 0.2) (layer F.Cu) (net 2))
 (segment (start 241.3 121.92) (end 239.725 121.92) (width 0.2) (layer F.Cu) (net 3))
 (segment (start 239.46 122.185) (end 233.12 122.185) (width 0.2) (layer F.Cu) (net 3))
 (segment (start 239.725 121.92) (end 239.46 122.185) (width 0.2) (layer F.Cu) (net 3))
 (segment (start 237.49 116.84) (end 241.3 116.84) (width 0.2) (layer F.Cu) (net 5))
 (segment (start 236.22 118.11) (end 237.49 116.84) (width 0.2) (layer F.Cu) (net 5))
 (segment (start 234.73 119.6) (end 236.22 118.11) (width 0.2) (layer F.Cu) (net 5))
 (segment (start 233.12 119.645) (end 233.6 119.645) (width 0.2) (layer F.Cu) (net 5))
 (segment (start 233.645 119.6) (end 234.73 119.6) (width 0.2) (layer F.Cu) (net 5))
 (segment (start 233.6 119.645) (end 233.645 119.6) (width 0.2) (layer F.Cu) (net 5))
 (segment (start 240.155 113.155) (end 241.3 114.3) (width 0.2) (layer F.Cu) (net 6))
 (segment (start 233.12 113.155) (end 240.155 113.155) (width 0.2) (layer F.Cu) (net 6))
 (segment (start 241.3 111.76) (end 240.097919 111.76) (width 0.2) (layer F.Cu) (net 7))
 (segment (start 239.972919 111.885) (end 233.12 111.885) (width 0.2) (layer F.Cu) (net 7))
 (segment (start 240.097919 111.76) (end 239.972919 111.885) (width 0.2) (layer F.Cu) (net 7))
 (segment (start 237.1875 106.68) (end 241.3 106.68) (width 0.2) (layer F.Cu) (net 9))
 (segment (start 236.22 107.6475) (end 237.1875 106.68) (width 0.2) (layer F.Cu) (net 9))
 (segment (start 234.3 109.345) (end 233.12 109.345) (width 0.2) (layer F.Cu) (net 9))
 (segment (start 236.22 107.6475) (end 235.9975 107.6475) (width 0.2) (layer F.Cu) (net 9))
 (segment (start 235.9975 107.6475) (end 234.3 109.345) (width 0.2) (layer F.Cu) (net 9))
 (segment (start 226.3825 110.6) (end 225.5825 109.8) (width 0.2) (layer F.Cu) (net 18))
 (segment (start 227.445 110.6) (end 226.3825 110.6) (width 0.2) (layer F.Cu) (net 18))
 (segment (start 228.17 110.615) (end 227.46 110.615) (width 0.2) (layer F.Cu) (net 18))
 (segment (start 227.46 110.615) (end 227.445 110.6) (width 0.2) (layer F.Cu) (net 18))
 (segment (start 228.055 112) (end 228.17 111.885) (width 0.2) (layer F.Cu) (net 16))
 (segment (start 225.5825 112) (end 228.055 112) (width 0.2) (layer F.Cu) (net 16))
 (segment (start 227.195 120.915) (end 228.17 120.915) (width 0.2) (layer F.Cu) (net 14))
 (segment (start 226.985 120.915) (end 227.195 120.915) (width 0.2) (layer F.Cu) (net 14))
 (segment (start 226.07 120) (end 226.985 120.915) (width 0.2) (layer F.Cu) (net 14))
 (segment (start 225.5825 120) (end 226.07 120) (width 0.2) (layer F.Cu) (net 14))
 (segment (start 228.155 122.2) (end 228.17 122.185) (width 0.2) (layer F.Cu) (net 12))
 (segment (start 225.5825 122.2) (end 228.155 122.2) (width 0.2) (layer F.Cu) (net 12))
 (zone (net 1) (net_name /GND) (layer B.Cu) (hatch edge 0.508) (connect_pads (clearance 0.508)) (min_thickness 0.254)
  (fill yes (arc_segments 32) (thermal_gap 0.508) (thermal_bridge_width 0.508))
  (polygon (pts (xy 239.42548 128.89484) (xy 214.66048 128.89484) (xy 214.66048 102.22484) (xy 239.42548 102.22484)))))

